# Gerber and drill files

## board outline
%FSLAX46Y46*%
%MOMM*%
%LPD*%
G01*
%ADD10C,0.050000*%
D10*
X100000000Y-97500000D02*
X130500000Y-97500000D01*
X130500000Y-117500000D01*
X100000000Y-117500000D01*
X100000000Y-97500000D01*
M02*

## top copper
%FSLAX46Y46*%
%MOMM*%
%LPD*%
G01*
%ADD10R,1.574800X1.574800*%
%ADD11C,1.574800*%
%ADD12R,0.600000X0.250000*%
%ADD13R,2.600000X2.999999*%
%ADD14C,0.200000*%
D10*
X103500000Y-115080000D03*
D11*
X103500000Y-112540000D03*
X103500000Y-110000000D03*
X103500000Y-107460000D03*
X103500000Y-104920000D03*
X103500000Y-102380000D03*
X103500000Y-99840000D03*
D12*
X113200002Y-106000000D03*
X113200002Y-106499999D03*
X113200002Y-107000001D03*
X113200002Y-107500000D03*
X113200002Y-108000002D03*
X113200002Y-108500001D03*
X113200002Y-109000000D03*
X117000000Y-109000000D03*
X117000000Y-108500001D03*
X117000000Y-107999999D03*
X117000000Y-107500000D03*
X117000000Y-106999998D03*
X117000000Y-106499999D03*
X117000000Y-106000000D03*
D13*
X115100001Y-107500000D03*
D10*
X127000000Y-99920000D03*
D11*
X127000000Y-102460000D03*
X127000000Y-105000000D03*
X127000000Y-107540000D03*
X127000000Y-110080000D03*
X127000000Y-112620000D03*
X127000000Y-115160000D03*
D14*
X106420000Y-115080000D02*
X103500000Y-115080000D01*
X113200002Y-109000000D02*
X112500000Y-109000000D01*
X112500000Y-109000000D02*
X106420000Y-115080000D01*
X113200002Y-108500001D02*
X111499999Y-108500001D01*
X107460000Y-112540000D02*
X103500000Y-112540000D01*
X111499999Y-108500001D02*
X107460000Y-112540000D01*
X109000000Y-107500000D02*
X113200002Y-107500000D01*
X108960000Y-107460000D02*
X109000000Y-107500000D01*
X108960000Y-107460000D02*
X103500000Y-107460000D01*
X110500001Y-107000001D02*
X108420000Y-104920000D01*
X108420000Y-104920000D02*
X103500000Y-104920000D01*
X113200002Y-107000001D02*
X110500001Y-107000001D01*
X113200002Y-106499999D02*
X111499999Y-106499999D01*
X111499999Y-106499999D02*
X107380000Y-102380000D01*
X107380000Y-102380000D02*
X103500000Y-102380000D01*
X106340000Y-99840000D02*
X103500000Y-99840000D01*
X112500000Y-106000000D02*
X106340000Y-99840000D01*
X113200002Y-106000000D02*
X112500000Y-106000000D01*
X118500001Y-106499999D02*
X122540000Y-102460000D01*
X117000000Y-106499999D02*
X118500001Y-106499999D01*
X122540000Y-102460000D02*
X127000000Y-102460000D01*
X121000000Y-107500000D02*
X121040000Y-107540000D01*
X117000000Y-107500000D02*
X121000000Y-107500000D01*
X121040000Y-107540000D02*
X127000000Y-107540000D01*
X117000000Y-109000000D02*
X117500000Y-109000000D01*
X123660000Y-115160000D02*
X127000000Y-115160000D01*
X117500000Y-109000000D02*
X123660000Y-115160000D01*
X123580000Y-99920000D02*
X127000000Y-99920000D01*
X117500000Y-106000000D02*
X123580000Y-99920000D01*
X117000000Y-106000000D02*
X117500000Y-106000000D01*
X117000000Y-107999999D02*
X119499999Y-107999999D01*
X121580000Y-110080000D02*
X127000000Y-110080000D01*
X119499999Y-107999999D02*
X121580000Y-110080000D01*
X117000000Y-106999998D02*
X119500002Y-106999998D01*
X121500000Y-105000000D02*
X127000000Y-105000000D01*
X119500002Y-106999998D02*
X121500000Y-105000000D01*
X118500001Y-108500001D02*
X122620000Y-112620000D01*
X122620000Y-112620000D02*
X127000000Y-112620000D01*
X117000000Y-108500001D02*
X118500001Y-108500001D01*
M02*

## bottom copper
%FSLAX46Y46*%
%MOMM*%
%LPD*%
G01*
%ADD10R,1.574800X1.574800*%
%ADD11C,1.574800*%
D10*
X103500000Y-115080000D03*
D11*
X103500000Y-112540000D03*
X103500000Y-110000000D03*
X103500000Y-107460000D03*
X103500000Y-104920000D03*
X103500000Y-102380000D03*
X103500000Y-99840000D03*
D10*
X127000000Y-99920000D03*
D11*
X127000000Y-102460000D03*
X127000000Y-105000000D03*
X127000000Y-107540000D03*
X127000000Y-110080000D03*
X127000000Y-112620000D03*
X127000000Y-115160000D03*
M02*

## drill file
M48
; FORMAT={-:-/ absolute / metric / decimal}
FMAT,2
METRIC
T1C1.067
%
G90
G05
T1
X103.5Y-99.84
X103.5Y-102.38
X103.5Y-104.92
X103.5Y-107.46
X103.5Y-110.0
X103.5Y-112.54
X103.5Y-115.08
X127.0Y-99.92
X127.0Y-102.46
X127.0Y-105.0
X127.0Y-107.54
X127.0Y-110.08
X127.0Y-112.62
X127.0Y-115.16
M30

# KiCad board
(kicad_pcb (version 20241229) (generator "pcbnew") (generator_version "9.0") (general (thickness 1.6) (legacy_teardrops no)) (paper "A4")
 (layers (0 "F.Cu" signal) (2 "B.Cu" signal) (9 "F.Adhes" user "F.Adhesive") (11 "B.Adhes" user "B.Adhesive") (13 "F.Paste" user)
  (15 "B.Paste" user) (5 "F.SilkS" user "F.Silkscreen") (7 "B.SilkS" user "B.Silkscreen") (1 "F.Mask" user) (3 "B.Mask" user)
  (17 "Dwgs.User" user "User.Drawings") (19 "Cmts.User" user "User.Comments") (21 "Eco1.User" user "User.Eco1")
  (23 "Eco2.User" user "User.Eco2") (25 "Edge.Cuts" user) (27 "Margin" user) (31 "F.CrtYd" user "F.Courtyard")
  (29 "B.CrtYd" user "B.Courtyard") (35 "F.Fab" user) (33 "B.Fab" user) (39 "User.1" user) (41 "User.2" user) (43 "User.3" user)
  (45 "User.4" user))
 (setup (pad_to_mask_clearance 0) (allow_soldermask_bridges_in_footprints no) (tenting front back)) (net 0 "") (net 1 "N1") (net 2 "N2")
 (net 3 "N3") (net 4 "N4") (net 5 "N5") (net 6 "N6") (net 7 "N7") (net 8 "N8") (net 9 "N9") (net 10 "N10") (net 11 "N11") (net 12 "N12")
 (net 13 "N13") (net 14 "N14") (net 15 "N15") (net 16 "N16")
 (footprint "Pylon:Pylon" (layer "F.Cu") (at 115 113.5)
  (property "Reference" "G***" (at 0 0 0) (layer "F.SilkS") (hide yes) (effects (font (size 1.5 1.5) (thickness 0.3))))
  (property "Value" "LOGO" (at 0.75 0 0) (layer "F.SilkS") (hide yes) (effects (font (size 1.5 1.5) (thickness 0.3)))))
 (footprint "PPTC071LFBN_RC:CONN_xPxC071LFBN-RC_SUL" (layer "F.Cu") (at 103.5 115.08 -90)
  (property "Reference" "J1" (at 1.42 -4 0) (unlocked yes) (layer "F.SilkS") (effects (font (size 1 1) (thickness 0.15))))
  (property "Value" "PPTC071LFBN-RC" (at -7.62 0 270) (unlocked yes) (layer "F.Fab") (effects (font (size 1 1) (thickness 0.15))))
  (pad "1" thru_hole rect (at 0 0 270) (size 1.5748 1.5748) (drill 1.0668) (layers "*.Cu" "*.Mask") (remove_unused_layers no) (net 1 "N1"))
  (pad "2" thru_hole circle (at -2.54 0 270) (size 1.5748 1.5748) (drill 1.0668) (layers "*.Cu" "*.Mask") (remove_unused_layers no)
   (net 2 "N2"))
  (pad "3" thru_hole circle (at -5.08 0 270) (size 1.5748 1.5748) (drill 1.0668) (layers "*.Cu" "*.Mask") (remove_unused_layers no)
   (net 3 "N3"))
  (pad "4" thru_hole circle (at -7.62 0 270) (size 1.5748 1.5748) (drill 1.0668) (layers "*.Cu" "*.Mask") (remove_unused_layers no)
   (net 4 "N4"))
  (pad "5" thru_hole circle (at -10.16 0 270) (size 1.5748 1.5748) (drill 1.0668) (layers "*.Cu" "*.Mask") (remove_unused_layers no)
   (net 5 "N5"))
  (pad "6" thru_hole circle (at -12.7 0 270) (size 1.5748 1.5748) (drill 1.0668) (layers "*.Cu" "*.Mask") (remove_unused_layers no)
   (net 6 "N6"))
  (pad "7" thru_hole circle (at -15.24 0 270) (size 1.5748 1.5748) (drill 1.0668) (layers "*.Cu" "*.Mask") (remove_unused_layers no)
   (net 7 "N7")))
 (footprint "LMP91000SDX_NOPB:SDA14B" (layer "F.Cu") (at 115.100001 107.5)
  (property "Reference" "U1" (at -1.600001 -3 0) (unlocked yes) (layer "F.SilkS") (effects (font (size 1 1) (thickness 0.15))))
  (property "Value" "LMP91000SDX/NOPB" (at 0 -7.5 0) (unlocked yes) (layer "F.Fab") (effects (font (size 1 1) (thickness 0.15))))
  (pad "1" smd rect (at -1.899999 -1.5) (size 0.6 0.25) (layers "F.Cu" "F.Mask") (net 7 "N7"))
  (pad "2" smd rect (at -1.899999 -1.000001) (size 0.6 0.25) (layers "F.Cu" "F.Mask") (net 6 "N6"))
  (pad "3" smd rect (at -1.899999 -0.499999) (size 0.6 0.25) (layers "F.Cu" "F.Mask") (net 5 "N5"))
  (pad "4" smd rect (at -1.899999 0) (size 0.6 0.25) (layers "F.Cu" "F.Mask") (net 4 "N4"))
  (pad "5" smd rect (at -1.899999 0.500002) (size 0.6 0.25) (layers "F.Cu" "F.Mask") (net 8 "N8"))
  (pad "6" smd rect (at -1.899999 1.000001) (size 0.6 0.25) (layers "F.Cu" "F.Mask") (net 2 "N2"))
  (pad "7" smd rect (at -1.899999 1.5) (size 0.6 0.25) (layers "F.Cu" "F.Mask") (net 1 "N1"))
  (pad "8" smd rect (at 1.899999 1.5) (size 0.6 0.25) (layers "F.Cu" "F.Mask") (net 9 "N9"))
  (pad "9" smd rect (at 1.899999 1.000001) (size 0.6 0.25) (layers "F.Cu" "F.Mask") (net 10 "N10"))
  (pad "10" smd rect (at 1.899999 0.499999) (size 0.6 0.25) (layers "F.Cu" "F.Mask") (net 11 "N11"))
  (pad "11" smd rect (at 1.899999 0) (size 0.6 0.25) (layers "F.Cu" "F.Mask") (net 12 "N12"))
  (pad "12" smd rect (at 1.899999 -0.500002) (size 0.6 0.25) (layers "F.Cu" "F.Mask") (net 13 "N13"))
  (pad "13" smd rect (at 1.899999 -1.000001) (size 0.6 0.25) (layers "F.Cu" "F.Mask") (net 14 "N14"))
  (pad "14" smd rect (at 1.899999 -1.5) (size 0.6 0.25) (layers "F.Cu" "F.Mask") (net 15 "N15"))
  (pad "15" smd rect (at 0 0) (size 2.6 2.999999) (layers "F.Cu" "F.Mask") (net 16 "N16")))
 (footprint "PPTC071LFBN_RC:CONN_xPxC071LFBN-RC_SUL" (layer "F.Cu") (at 127 99.92 90)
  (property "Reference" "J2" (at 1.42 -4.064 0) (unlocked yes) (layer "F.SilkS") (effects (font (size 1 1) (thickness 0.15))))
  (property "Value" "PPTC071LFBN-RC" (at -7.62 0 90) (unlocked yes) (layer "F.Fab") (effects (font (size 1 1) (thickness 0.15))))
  (pad "1" thru_hole rect (at 0 0 90) (size 1.5748 1.5748) (drill 1.0668) (layers "*.Cu" "*.Mask") (remove_unused_layers no) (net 15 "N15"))
  (pad "2" thru_hole circle (at -2.54 0 90) (size 1.5748 1.5748) (drill 1.0668) (layers "*.Cu" "*.Mask") (remove_unused_layers no)
   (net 14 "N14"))
  (pad "3" thru_hole circle (at -5.08 0 90) (size 1.5748 1.5748) (drill 1.0668) (layers "*.Cu" "*.Mask") (remove_unused_layers no)
   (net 13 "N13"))
  (pad "4" thru_hole circle (at -7.62 0 90) (size 1.5748 1.5748) (drill 1.0668) (layers "*.Cu" "*.Mask") (remove_unused_layers no)
   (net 12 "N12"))
  (pad "5" thru_hole circle (at -10.16 0 90) (size 1.5748 1.5748) (drill 1.0668) (layers "*.Cu" "*.Mask") (remove_unused_layers no)
   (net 11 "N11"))
  (pad "6" thru_hole circle (at -12.7 0 90) (size 1.5748 1.5748) (drill 1.0668) (layers "*.Cu" "*.Mask") (remove_unused_layers no)
   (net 10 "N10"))
  (pad "7" thru_hole circle (at -15.24 0 90) (size 1.5748 1.5748) (drill 1.0668) (layers "*.Cu" "*.Mask") (remove_unused_layers no)
   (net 9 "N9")))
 (gr_rect (start 100 97.5) (end 130.5 117.5) (stroke (width 0.05) (type solid)) (fill no) (layer "Edge.Cuts"))
 (segment (start 106.42 115.08) (end 103.5 115.08) (width 0.2) (layer "F.Cu") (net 1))
 (segment (start 113.200002 109) (end 112.5 109) (width 0.2) (layer "F.Cu") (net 1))
 (segment (start 112.5 109) (end 106.42 115.08) (width 0.2) (layer "F.Cu") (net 1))
 (segment (start 113.200002 108.500001) (end 111.499999 108.500001) (width 0.2) (layer "F.Cu") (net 2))
 (segment (start 107.46 112.54) (end 103.5 112.54) (width 0.2) (layer "F.Cu") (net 2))
 (segment (start 111.499999 108.500001) (end 107.46 112.54) (width 0.2) (layer "F.Cu") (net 2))
 (segment (start 109 107.5) (end 113.200002 107.5) (width 0.2) (layer "F.Cu") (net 4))
 (segment (start 108.96 107.46) (end 109 107.5) (width 0.2) (layer "F.Cu") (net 4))
 (segment (start 108.96 107.46) (end 103.5 107.46) (width 0.2) (layer "F.Cu") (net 4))
 (segment (start 110.500001 107.000001) (end 108.42 104.92) (width 0.2) (layer "F.Cu") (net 5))
 (segment (start 108.42 104.92) (end 103.5 104.92) (width 0.2) (layer "F.Cu") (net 5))
 (segment (start 113.200002 107.000001) (end 110.500001 107.000001) (width 0.2) (layer "F.Cu") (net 5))
 (segment (start 113.200002 106.499999) (end 111.499999 106.499999) (width 0.2) (layer "F.Cu") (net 6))
 (segment (start 111.499999 106.499999) (end 107.38 102.38) (width 0.2) (layer "F.Cu") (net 6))
 (segment (start 107.38 102.38) (end 103.5 102.38) (width 0.2) (layer "F.Cu") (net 6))
 (segment (start 106.34 99.84) (end 103.5 99.84) (width 0.2) (layer "F.Cu") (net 7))
 (segment (start 112.5 106) (end 106.34 99.84) (width 0.2) (layer "F.Cu") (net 7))
 (segment (start 113.200002 106) (end 112.5 106) (width 0.2) (layer "F.Cu") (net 7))
 (segment (start 118.500001 106.499999) (end 122.54 102.46) (width 0.2) (layer "F.Cu") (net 14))
 (segment (start 117 106.499999) (end 118.500001 106.499999) (width 0.2) (layer "F.Cu") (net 14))
 (segment (start 122.54 102.46) (end 127 102.46) (width 0.2) (layer "F.Cu") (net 14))
 (segment (start 121 107.5) (end 121.04 107.54) (width 0.2) (layer "F.Cu") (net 12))
 (segment (start 117 107.5) (end 121 107.5) (width 0.2) (layer "F.Cu") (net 12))
 (segment (start 121.04 107.54) (end 127 107.54) (width 0.2) (layer "F.Cu") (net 12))
 (segment (start 117 109) (end 117.5 109) (width 0.2) (layer "F.Cu") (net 9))
 (segment (start 123.66 115.16) (end 127 115.16) (width 0.2) (layer "F.Cu") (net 9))
 (segment (start 117.5 109) (end 123.66 115.16) (width 0.2) (layer "F.Cu") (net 9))
 (segment (start 123.58 99.92) (end 127 99.92) (width 0.2) (layer "F.Cu") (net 15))
 (segment (start 117.5 106) (end 123.58 99.92) (width 0.2) (layer "F.Cu") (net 15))
 (segment (start 117 106) (end 117.5 106) (width 0.2) (layer "F.Cu") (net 15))
 (segment (start 117 107.999999) (end 119.499999 107.999999) (width 0.2) (layer "F.Cu") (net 11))
 (segment (start 121.58 110.08) (end 127 110.08) (width 0.2) (layer "F.Cu") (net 11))
 (segment (start 119.499999 107.999999) (end 121.58 110.08) (width 0.2) (layer "F.Cu") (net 11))
 (segment (start 117 106.999998) (end 119.500002 106.999998) (width 0.2) (layer "F.Cu") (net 13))
 (segment (start 121.5 105) (end 127 105) (width 0.2) (layer "F.Cu") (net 13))
 (segment (start 119.500002 106.999998) (end 121.5 105) (width 0.2) (layer "F.Cu") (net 13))
 (segment (start 118.500001 108.500001) (end 122.62 112.62) (width 0.2) (layer "F.Cu") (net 10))
 (segment (start 122.62 112.62) (end 127 112.62) (width 0.2) (layer "F.Cu") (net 10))
 (segment (start 117 108.500001) (end 118.500001 108.500001) (width 0.2) (layer "F.Cu") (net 10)))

